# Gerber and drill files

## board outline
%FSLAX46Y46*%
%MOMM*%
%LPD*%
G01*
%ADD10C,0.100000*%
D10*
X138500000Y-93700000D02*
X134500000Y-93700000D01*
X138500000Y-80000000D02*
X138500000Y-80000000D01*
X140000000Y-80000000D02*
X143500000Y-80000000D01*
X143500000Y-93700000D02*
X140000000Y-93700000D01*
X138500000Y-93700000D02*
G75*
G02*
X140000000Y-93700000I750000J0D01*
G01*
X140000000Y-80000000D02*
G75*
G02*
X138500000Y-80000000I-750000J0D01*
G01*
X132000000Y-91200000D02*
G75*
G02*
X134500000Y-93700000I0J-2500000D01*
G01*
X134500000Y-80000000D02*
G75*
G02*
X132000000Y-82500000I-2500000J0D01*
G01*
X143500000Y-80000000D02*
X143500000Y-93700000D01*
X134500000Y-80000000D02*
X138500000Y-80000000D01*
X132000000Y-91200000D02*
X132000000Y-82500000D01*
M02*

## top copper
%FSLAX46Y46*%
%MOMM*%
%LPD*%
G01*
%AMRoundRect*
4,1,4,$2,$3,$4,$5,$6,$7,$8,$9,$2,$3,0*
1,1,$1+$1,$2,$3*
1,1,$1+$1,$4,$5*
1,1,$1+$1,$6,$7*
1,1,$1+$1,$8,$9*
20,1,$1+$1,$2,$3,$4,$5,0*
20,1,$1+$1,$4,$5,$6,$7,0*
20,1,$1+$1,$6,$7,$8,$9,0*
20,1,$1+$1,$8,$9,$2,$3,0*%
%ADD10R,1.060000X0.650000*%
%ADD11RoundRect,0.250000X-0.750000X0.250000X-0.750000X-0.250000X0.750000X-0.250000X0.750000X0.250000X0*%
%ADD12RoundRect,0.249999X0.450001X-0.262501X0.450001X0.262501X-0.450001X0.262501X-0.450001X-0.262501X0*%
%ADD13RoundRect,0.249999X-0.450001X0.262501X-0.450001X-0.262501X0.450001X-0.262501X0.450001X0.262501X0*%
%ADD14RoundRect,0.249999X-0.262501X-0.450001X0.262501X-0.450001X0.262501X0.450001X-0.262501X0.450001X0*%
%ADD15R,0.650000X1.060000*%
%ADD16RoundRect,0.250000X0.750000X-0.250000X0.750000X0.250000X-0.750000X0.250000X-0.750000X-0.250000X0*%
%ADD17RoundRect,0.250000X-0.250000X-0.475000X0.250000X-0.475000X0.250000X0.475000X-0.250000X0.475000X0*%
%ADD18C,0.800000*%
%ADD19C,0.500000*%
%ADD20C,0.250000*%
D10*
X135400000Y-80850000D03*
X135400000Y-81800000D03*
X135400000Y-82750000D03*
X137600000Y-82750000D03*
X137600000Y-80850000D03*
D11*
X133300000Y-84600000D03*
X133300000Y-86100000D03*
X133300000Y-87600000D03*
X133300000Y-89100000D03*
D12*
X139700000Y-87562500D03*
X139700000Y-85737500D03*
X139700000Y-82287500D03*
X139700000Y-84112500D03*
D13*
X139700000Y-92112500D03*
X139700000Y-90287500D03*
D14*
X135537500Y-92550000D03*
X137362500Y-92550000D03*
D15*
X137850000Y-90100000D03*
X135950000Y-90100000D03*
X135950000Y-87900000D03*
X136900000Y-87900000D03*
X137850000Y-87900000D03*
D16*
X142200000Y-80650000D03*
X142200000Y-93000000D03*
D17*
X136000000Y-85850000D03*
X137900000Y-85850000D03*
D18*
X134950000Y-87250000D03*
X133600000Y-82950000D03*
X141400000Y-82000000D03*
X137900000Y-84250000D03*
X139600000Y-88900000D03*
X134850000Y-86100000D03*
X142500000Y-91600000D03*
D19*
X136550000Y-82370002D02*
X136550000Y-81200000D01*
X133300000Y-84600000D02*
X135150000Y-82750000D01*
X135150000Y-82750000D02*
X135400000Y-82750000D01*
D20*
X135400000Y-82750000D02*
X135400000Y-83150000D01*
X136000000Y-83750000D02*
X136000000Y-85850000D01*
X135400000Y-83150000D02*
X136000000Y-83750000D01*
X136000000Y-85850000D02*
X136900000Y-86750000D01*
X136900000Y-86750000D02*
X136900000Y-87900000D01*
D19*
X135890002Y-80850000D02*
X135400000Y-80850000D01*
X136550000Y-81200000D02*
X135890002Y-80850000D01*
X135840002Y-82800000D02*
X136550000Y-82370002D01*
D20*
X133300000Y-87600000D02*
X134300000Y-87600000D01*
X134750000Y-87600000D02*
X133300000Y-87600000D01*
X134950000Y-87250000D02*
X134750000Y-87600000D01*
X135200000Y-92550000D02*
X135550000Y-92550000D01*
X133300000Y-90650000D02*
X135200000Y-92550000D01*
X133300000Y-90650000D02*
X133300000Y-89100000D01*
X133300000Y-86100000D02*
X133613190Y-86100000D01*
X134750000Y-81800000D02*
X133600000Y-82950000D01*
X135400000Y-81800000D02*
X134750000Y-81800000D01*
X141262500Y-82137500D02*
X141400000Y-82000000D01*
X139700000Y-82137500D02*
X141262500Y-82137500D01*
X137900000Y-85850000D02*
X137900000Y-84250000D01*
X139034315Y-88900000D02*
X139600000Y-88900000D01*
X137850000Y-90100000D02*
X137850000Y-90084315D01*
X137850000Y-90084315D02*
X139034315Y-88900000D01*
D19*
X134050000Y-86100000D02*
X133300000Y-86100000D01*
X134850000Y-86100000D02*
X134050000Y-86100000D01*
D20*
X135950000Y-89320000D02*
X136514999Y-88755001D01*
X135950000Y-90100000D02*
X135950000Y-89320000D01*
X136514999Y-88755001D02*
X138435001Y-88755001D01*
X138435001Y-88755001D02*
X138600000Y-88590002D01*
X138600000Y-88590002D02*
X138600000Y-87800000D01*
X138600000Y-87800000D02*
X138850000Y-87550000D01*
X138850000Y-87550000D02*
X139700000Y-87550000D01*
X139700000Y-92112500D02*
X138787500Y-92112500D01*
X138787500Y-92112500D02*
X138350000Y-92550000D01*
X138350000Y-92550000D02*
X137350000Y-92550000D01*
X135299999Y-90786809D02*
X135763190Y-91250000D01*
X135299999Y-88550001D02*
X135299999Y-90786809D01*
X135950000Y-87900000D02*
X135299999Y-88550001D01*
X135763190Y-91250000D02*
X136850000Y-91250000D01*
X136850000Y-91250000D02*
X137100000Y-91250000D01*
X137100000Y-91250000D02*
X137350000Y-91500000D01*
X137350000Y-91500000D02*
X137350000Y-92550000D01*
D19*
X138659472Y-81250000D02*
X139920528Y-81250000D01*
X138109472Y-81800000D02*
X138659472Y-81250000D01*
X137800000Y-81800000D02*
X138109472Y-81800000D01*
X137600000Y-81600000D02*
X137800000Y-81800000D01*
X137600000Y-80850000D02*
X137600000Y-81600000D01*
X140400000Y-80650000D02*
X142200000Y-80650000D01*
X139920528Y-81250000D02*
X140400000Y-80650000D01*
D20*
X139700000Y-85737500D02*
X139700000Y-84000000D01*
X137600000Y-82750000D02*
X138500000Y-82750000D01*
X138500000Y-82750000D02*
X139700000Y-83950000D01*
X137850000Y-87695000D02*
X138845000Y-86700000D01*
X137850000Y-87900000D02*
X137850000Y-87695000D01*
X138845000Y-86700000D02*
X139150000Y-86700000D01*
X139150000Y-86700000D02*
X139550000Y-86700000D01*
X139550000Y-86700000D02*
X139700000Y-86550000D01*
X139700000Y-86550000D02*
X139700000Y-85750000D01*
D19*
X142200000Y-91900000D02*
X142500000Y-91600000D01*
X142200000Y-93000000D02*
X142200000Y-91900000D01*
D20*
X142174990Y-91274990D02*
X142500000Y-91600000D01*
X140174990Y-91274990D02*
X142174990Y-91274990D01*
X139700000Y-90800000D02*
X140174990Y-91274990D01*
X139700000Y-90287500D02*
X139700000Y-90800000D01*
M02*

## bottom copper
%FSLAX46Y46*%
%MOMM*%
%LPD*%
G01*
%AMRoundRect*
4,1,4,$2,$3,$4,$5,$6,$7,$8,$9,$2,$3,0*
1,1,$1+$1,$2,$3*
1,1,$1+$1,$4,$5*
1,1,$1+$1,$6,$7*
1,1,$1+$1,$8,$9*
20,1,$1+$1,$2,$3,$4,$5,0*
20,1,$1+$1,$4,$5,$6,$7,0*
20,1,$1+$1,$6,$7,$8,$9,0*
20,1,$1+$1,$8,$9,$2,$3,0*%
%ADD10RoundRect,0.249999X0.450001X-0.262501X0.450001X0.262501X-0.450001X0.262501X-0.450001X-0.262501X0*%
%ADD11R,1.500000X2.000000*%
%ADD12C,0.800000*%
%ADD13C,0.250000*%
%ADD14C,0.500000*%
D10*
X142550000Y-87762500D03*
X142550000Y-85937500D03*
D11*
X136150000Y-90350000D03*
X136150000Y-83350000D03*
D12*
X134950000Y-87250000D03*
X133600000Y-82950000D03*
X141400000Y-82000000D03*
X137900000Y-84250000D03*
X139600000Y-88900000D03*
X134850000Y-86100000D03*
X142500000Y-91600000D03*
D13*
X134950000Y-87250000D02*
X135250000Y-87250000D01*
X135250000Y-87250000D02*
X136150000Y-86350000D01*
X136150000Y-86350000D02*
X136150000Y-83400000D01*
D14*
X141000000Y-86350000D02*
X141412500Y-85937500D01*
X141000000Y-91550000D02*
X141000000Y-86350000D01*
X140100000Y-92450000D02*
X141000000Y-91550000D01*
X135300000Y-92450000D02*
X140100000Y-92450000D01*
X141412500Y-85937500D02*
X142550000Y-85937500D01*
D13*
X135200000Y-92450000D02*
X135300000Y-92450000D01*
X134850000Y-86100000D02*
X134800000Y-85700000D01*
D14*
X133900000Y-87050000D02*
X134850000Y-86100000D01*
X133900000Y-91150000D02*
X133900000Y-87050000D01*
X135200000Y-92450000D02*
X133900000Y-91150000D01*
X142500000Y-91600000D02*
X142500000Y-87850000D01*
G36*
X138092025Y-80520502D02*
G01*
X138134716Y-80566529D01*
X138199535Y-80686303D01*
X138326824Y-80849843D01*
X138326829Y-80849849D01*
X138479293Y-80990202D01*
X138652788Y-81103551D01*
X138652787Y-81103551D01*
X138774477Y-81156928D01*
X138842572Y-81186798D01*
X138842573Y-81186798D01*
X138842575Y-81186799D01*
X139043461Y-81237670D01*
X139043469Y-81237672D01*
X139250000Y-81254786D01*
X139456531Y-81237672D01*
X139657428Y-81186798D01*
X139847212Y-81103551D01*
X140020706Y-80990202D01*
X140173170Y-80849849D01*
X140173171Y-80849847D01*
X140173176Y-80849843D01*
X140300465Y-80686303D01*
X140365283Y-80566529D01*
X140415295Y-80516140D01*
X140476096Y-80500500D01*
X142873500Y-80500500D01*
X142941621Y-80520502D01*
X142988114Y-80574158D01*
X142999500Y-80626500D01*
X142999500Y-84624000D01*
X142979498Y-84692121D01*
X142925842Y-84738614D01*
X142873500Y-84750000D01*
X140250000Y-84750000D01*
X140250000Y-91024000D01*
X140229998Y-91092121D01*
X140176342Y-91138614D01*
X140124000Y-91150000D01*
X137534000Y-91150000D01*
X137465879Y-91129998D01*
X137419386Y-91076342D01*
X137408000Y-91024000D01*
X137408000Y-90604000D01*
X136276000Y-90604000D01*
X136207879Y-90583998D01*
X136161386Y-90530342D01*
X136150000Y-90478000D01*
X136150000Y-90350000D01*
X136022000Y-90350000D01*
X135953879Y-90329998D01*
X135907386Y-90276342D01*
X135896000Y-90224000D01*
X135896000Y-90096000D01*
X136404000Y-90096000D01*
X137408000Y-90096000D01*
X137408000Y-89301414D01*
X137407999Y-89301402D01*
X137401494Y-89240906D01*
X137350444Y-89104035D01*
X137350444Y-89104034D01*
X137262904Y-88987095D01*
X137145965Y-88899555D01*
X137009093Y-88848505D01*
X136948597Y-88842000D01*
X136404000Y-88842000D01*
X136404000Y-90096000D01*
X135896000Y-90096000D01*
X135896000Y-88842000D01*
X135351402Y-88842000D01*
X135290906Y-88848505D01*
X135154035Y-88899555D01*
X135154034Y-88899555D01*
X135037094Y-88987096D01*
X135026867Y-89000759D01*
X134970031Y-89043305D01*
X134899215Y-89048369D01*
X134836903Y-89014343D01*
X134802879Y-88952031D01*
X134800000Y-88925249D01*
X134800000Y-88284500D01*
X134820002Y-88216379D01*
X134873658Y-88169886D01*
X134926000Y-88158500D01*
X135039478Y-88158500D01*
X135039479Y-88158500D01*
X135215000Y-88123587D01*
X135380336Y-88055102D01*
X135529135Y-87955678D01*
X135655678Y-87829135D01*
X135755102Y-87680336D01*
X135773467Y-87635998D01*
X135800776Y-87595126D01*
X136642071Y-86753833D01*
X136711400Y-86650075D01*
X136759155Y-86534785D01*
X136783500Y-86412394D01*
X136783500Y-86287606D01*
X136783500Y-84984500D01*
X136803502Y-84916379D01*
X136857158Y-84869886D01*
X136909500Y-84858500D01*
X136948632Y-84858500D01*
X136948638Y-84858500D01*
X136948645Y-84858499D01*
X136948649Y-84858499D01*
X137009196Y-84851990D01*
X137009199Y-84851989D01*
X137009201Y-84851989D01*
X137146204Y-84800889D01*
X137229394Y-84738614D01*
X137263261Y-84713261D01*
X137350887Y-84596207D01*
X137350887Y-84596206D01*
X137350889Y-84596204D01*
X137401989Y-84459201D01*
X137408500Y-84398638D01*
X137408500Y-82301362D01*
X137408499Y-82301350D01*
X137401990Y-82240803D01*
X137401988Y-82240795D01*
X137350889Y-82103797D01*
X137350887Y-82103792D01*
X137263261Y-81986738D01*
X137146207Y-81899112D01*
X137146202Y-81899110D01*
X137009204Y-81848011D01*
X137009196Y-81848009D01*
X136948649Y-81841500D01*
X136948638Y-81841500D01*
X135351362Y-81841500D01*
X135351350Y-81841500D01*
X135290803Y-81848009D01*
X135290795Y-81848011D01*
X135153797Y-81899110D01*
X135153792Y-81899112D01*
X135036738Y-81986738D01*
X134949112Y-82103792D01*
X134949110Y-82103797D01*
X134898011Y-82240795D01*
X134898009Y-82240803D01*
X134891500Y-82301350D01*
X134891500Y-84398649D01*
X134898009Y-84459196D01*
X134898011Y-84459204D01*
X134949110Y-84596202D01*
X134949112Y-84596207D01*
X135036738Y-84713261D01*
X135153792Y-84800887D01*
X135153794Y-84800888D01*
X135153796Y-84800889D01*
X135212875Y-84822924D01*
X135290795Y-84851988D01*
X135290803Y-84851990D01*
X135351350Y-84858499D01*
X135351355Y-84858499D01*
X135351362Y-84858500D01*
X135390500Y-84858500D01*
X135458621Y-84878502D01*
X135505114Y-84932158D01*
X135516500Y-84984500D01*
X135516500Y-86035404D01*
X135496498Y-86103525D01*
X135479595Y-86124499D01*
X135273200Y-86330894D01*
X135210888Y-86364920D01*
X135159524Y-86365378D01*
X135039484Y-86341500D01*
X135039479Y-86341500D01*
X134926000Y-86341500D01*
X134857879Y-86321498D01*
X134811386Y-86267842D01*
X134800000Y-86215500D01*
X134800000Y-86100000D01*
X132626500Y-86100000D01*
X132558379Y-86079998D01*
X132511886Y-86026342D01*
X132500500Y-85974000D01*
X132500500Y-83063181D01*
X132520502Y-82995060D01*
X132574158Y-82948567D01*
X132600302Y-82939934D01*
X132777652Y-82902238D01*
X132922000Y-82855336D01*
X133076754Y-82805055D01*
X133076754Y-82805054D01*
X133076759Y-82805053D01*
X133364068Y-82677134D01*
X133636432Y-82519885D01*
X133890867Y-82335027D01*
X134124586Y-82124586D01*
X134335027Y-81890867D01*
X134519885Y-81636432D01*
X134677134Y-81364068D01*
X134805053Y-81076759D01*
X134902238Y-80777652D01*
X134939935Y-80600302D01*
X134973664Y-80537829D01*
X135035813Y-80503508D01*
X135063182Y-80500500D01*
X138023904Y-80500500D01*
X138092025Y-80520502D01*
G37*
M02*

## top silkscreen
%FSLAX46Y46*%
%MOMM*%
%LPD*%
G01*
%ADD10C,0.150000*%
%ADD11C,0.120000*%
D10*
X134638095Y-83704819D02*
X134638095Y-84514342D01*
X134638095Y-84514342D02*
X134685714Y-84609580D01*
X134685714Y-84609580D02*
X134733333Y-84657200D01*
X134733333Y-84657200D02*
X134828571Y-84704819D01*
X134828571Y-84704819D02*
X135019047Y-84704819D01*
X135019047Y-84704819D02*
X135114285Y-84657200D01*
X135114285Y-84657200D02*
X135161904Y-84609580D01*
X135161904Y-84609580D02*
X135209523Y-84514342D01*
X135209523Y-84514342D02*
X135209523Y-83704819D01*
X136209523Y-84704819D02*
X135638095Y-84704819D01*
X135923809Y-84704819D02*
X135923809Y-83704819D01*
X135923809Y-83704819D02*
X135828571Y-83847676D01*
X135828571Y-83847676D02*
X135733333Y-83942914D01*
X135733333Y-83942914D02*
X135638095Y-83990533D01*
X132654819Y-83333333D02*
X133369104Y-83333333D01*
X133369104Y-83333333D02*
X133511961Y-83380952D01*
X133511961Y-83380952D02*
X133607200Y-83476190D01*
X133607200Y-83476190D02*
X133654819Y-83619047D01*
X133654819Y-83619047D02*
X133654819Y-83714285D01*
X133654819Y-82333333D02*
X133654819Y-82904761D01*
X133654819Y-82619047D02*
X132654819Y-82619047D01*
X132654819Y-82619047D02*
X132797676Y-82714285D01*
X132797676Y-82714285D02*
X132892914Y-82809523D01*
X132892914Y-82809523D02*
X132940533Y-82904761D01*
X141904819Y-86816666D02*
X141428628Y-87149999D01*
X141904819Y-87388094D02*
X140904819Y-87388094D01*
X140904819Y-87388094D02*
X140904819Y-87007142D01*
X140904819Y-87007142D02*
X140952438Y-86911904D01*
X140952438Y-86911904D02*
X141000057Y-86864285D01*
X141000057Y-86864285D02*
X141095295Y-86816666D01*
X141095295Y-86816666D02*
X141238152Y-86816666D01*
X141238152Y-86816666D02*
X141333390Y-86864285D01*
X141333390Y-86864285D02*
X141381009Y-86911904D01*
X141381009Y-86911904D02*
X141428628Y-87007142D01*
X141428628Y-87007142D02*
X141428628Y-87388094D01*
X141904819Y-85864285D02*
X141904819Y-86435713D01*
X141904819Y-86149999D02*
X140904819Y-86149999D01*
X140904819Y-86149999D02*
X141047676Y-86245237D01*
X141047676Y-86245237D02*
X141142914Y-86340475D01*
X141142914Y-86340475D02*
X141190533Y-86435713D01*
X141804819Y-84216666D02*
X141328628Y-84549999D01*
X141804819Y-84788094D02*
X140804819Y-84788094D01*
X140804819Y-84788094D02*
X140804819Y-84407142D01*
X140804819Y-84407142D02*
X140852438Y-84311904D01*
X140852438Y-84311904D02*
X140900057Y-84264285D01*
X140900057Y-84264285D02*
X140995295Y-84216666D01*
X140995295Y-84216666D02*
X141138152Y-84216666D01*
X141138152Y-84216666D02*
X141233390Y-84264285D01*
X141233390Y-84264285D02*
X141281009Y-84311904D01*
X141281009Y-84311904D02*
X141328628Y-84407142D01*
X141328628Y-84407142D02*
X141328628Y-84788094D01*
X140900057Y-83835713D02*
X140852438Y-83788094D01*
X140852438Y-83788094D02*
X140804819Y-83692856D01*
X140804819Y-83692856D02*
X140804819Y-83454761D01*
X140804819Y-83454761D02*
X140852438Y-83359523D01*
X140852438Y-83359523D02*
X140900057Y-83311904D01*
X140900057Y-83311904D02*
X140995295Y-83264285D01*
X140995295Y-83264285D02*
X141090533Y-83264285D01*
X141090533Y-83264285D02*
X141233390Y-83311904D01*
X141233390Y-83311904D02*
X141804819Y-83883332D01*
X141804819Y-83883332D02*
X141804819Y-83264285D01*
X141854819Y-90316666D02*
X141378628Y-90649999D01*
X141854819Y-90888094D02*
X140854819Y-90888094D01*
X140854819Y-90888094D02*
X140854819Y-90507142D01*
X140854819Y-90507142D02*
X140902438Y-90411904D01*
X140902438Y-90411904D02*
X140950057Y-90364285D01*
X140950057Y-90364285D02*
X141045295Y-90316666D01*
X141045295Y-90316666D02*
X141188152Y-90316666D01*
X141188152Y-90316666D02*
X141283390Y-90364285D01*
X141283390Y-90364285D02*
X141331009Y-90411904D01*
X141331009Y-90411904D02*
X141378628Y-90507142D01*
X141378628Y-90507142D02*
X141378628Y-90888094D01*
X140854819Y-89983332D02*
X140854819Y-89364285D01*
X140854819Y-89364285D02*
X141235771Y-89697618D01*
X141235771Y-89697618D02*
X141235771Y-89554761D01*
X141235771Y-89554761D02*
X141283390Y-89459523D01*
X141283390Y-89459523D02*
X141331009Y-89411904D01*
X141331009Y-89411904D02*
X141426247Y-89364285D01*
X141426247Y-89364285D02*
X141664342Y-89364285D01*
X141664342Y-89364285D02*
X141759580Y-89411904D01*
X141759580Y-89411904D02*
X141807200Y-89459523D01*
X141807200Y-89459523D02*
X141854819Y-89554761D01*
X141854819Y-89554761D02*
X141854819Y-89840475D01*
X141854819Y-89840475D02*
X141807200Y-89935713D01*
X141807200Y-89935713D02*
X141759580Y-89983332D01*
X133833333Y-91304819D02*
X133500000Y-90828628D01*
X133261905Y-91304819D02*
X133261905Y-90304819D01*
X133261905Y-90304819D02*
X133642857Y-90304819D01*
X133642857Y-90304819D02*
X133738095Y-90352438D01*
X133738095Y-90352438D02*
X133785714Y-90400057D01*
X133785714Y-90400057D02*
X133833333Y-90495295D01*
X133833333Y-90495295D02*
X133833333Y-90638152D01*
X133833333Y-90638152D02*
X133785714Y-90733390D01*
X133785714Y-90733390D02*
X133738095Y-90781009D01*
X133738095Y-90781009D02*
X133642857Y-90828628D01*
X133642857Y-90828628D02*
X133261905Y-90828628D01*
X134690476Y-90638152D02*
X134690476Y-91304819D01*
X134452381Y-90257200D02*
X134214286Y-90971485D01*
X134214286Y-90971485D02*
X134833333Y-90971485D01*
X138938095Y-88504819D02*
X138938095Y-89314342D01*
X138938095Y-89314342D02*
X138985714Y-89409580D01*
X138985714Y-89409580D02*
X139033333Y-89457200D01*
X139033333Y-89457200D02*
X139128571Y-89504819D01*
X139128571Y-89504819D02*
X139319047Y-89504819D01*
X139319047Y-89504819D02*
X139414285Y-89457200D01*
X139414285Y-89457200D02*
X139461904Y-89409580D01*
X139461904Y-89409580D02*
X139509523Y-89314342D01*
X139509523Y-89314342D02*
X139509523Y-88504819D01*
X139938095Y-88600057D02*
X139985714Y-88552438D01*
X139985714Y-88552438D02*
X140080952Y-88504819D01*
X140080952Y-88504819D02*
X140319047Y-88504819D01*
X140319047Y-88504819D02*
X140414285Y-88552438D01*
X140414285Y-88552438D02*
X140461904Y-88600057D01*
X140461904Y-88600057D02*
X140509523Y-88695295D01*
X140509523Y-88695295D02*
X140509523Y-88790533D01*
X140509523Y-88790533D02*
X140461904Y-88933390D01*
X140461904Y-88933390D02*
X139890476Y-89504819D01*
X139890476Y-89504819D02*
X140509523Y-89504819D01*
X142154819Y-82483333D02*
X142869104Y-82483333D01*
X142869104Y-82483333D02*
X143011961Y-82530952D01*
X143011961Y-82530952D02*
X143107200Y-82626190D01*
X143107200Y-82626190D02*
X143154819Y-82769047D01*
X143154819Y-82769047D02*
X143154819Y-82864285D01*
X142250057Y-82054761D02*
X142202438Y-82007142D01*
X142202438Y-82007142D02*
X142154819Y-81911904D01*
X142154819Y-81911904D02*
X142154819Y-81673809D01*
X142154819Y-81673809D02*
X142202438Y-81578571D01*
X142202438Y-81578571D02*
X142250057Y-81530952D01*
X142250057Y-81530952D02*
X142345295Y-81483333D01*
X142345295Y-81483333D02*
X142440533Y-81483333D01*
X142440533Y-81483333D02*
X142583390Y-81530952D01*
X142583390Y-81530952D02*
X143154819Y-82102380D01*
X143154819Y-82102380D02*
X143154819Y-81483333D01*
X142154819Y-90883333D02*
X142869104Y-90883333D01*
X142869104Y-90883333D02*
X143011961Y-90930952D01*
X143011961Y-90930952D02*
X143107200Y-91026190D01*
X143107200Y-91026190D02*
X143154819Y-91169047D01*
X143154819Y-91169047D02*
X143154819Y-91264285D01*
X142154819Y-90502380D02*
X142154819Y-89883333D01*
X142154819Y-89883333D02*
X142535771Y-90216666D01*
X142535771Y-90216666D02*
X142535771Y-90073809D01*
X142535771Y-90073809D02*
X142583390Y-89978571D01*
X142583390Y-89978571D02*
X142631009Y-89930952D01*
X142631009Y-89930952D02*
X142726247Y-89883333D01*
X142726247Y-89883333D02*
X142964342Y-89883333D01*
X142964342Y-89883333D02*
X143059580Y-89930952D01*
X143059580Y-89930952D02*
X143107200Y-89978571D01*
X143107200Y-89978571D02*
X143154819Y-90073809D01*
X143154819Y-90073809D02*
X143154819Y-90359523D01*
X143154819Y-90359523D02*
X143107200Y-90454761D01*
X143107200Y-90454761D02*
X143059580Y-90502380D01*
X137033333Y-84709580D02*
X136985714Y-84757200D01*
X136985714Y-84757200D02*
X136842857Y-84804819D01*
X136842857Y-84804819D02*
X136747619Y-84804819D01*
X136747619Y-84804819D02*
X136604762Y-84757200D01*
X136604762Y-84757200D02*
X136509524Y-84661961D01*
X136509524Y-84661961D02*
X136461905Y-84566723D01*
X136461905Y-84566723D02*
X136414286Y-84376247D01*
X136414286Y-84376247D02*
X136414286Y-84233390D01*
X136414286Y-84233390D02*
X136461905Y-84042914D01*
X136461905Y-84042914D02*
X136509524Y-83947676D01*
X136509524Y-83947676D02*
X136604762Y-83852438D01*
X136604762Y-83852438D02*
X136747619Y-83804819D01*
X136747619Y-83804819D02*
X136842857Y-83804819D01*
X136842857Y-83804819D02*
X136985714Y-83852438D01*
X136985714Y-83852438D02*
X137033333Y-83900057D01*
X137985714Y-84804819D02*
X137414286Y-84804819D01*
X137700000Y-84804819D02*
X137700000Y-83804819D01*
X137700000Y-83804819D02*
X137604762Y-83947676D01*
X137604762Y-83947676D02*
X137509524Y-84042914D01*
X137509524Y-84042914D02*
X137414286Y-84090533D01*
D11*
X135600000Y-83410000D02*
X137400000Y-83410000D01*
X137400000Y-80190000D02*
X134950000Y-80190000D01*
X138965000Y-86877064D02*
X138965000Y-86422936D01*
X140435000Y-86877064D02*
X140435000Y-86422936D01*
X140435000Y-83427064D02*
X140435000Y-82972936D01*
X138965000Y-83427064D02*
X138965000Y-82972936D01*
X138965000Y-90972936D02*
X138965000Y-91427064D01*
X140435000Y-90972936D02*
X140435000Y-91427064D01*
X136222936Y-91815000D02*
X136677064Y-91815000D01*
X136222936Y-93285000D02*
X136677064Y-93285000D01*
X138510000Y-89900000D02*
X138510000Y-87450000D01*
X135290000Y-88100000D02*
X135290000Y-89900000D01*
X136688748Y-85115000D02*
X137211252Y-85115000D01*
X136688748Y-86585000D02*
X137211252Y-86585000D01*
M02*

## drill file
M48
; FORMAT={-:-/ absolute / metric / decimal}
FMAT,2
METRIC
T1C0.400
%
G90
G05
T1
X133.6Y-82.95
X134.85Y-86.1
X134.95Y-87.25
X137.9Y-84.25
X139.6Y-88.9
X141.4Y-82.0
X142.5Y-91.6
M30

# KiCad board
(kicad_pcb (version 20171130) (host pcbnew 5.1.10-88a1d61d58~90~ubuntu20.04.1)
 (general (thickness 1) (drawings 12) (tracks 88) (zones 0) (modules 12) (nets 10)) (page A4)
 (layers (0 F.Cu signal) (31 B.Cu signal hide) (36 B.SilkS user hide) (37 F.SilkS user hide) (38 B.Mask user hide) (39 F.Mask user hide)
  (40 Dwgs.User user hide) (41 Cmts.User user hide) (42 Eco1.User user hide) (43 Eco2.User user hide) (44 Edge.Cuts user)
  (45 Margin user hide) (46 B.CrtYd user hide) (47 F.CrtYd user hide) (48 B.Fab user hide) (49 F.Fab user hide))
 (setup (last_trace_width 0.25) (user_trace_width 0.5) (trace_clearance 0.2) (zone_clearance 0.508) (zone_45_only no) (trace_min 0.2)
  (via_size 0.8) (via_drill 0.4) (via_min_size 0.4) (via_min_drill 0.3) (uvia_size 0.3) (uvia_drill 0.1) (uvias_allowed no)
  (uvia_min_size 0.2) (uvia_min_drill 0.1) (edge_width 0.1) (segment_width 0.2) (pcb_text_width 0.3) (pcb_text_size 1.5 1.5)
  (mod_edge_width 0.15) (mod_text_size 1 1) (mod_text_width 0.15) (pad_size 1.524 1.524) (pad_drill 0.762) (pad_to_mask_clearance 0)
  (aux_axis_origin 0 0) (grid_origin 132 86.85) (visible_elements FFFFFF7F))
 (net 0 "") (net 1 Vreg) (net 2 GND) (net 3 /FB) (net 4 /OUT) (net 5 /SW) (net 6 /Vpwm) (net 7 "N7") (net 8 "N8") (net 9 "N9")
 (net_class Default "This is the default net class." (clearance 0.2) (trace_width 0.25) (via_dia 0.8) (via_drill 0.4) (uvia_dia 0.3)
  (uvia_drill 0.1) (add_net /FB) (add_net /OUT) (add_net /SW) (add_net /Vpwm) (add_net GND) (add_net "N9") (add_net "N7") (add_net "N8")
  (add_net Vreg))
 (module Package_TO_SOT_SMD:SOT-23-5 (layer F.Cu) (at 136.5 81.8)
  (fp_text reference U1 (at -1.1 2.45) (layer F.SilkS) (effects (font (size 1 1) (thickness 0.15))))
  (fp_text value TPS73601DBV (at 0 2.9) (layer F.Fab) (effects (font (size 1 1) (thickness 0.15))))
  (fp_line (start -0.9 1.61) (end 0.9 1.61) (layer F.SilkS) (width 0.12))
  (fp_line (start 0.9 -1.61) (end -1.55 -1.61) (layer F.SilkS) (width 0.12))
  (pad 1 smd rect (at -1.1 -0.95) (size 1.06 0.65) (layers F.Cu F.Paste F.Mask) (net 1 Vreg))
  (pad 2 smd rect (at -1.1 0) (size 1.06 0.65) (layers F.Cu F.Paste F.Mask) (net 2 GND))
  (pad 3 smd rect (at -1.1 0.95) (size 1.06 0.65) (layers F.Cu F.Paste F.Mask) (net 1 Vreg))
  (pad 4 smd rect (at 1.1 0.95) (size 1.06 0.65) (layers F.Cu F.Paste F.Mask) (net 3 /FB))
  (pad 5 smd rect (at 1.1 -0.95) (size 1.06 0.65) (layers F.Cu F.Paste F.Mask) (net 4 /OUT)))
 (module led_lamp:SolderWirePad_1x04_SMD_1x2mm (layer F.Cu) (at 133.3 84.6 270)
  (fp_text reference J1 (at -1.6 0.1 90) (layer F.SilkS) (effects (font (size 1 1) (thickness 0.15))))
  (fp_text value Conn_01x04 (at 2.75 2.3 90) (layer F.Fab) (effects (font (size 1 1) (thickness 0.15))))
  (pad 1 smd roundrect (at 0 0 270) (size 1 2) (layers F.Cu F.Paste F.Mask) (roundrect_rratio 0.25) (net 1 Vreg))
  (pad 2 smd roundrect (at 1.5 0 270) (size 1 2) (layers F.Cu F.Paste F.Mask) (roundrect_rratio 0.25) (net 2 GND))
  (pad 3 smd roundrect (at 3 0 270) (size 1 2) (layers F.Cu F.Paste F.Mask) (roundrect_rratio 0.25) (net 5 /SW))
  (pad 4 smd roundrect (at 4.5 0 270) (size 1 2) (layers F.Cu F.Paste F.Mask) (roundrect_rratio 0.25) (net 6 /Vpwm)))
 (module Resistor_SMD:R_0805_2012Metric (layer F.Cu) (at 139.7 86.65 90)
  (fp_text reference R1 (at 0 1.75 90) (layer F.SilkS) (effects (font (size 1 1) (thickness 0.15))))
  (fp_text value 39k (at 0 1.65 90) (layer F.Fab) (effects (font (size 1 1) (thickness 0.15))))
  (fp_line (start -0.227064 -0.735) (end 0.227064 -0.735) (layer F.SilkS) (width 0.12))
  (fp_line (start -0.227064 0.735) (end 0.227064 0.735) (layer F.SilkS) (width 0.12))
  (pad 1 smd roundrect (at -0.9125 0 90) (size 1.025 1.4) (layers F.Cu F.Paste F.Mask) (roundrect_rratio 0.2439014634146341) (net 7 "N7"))
  (pad 2 smd roundrect (at 0.9125 0 90) (size 1.025 1.4) (layers F.Cu F.Paste F.Mask) (roundrect_rratio 0.2439014634146341) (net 3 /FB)))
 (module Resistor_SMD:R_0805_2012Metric (layer F.Cu) (at 139.7 83.2 90)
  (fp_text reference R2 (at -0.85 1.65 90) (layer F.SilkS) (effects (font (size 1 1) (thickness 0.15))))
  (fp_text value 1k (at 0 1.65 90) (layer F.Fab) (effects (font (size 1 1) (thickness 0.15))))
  (fp_line (start -0.227064 0.735) (end 0.227064 0.735) (layer F.SilkS) (width 0.12))
  (fp_line (start -0.227064 -0.735) (end 0.227064 -0.735) (layer F.SilkS) (width 0.12))
  (pad 2 smd roundrect (at 0.9125 0 90) (size 1.025 1.4) (layers F.Cu F.Paste F.Mask) (roundrect_rratio 0.2439014634146341) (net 2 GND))
  (pad 1 smd roundrect (at -0.9125 0 90) (size 1.025 1.4) (layers F.Cu F.Paste F.Mask) (roundrect_rratio 0.2439014634146341) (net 3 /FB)))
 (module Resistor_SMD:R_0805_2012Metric (layer F.Cu) (at 139.7 91.2 270)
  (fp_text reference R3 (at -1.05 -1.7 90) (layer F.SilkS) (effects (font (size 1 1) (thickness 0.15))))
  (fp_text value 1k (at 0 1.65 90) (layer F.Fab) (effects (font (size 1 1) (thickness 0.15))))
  (fp_line (start -0.227064 0.735) (end 0.227064 0.735) (layer F.SilkS) (width 0.12))
  (fp_line (start -0.227064 -0.735) (end 0.227064 -0.735) (layer F.SilkS) (width 0.12))
  (pad 2 smd roundrect (at 0.9125 0 270) (size 1.025 1.4) (layers F.Cu F.Paste F.Mask) (roundrect_rratio 0.2439014634146341) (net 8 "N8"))
  (pad 1 smd roundrect (at -0.9125 0 270) (size 1.025 1.4) (layers F.Cu F.Paste F.Mask) (roundrect_rratio 0.2439014634146341) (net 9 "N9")))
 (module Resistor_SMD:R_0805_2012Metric (layer F.Cu) (at 136.45 92.55)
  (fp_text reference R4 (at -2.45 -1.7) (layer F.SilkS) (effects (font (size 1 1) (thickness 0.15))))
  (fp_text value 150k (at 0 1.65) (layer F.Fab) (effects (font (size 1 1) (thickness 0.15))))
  (fp_line (start -0.227064 -0.735) (end 0.227064 -0.735) (layer F.SilkS) (width 0.12))
  (fp_line (start -0.227064 0.735) (end 0.227064 0.735) (layer F.SilkS) (width 0.12))
  (pad 1 smd roundrect (at -0.9125 0) (size 1.025 1.4) (layers F.Cu F.Paste F.Mask) (roundrect_rratio 0.2439014634146341) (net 6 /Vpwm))
  (pad 2 smd roundrect (at 0.9125 0) (size 1.025 1.4) (layers F.Cu F.Paste F.Mask) (roundrect_rratio 0.2439014634146341) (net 8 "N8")))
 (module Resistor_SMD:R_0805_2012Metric (layer B.Cu) (at 142.55 86.85 90)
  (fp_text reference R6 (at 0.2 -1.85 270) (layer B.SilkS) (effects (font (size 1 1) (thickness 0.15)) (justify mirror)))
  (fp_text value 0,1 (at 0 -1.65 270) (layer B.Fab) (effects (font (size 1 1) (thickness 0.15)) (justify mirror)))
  (pad 1 smd roundrect (at -0.9125 0 90) (size 1.025 1.4) (layers B.Cu B.Paste B.Mask) (roundrect_rratio 0.2439014634146341) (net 9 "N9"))
  (pad 2 smd roundrect (at 0.9125 0 90) (size 1.025 1.4) (layers B.Cu B.Paste B.Mask) (roundrect_rratio 0.2439014634146341) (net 2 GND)))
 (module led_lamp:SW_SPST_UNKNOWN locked (layer B.Cu) (at 136.15 86.85 90)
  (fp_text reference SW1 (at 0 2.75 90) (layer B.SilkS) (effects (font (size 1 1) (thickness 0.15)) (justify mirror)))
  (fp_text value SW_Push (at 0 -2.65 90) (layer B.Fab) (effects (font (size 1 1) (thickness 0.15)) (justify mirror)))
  (pad 1 smd rect (at -3.5 0 90) (size 2 1.5) (layers B.Cu B.Paste B.Mask) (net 2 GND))
  (pad 2 smd rect (at 3.5 0 90) (size 2 1.5) (layers B.Cu B.Paste B.Mask) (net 5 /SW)))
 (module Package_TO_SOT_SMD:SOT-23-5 (layer F.Cu) (at 136.9 89 270)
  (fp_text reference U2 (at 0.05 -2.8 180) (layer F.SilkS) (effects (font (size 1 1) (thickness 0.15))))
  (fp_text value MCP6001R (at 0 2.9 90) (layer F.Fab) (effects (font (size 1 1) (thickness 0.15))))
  (fp_line (start 0.9 -1.61) (end -1.55 -1.61) (layer F.SilkS) (width 0.12))
  (fp_line (start -0.9 1.61) (end 0.9 1.61) (layer F.SilkS) (width 0.12))
  (pad 5 smd rect (at 1.1 -0.95 270) (size 1.06 0.65) (layers F.Cu F.Paste F.Mask) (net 2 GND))
  (pad 4 smd rect (at 1.1 0.95 270) (size 1.06 0.65) (layers F.Cu F.Paste F.Mask) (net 7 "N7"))
  (pad 3 smd rect (at -1.1 0.95 270) (size 1.06 0.65) (layers F.Cu F.Paste F.Mask) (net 8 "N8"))
  (pad 2 smd rect (at -1.1 0 270) (size 1.06 0.65) (layers F.Cu F.Paste F.Mask) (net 1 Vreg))
  (pad 1 smd rect (at -1.1 -0.95 270) (size 1.06 0.65) (layers F.Cu F.Paste F.Mask) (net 3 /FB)))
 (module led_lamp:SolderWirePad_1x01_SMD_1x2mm (layer F.Cu) (at 142.2 80.65 90)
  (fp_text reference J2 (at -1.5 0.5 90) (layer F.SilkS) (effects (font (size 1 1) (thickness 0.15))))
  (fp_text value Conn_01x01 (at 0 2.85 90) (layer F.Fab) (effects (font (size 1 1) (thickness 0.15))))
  (pad 1 smd roundrect (at 0 0 90) (size 1 2) (layers F.Cu F.Paste F.Mask) (roundrect_rratio 0.25) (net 4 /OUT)))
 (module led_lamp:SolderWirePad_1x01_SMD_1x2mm (layer F.Cu) (at 142.2 93 90)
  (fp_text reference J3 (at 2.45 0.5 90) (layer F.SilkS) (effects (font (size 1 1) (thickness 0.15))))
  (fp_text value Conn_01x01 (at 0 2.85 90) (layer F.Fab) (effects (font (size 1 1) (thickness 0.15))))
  (pad 1 smd roundrect (at 0 0 90) (size 1 2) (layers F.Cu F.Paste F.Mask) (roundrect_rratio 0.25) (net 9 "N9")))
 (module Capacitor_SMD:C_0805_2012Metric (layer F.Cu) (at 136.95 85.85)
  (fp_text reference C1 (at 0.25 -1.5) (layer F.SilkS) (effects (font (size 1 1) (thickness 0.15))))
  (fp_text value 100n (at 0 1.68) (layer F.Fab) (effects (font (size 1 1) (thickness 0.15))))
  (fp_line (start -0.261252 -0.735) (end 0.261252 -0.735) (layer F.SilkS) (width 0.12))
  (fp_line (start -0.261252 0.735) (end 0.261252 0.735) (layer F.SilkS) (width 0.12))
  (pad 1 smd roundrect (at -0.95 0) (size 1 1.45) (layers F.Cu F.Paste F.Mask) (roundrect_rratio 0.25) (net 1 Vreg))
  (pad 2 smd roundrect (at 0.95 0) (size 1 1.45) (layers F.Cu F.Paste F.Mask) (roundrect_rratio 0.25) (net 2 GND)))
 (gr_line (start 138.5 93.7) (end 134.5 93.7) (layer Edge.Cuts) (width 0.1))
 (gr_line (start 138.5 80) (end 138.5 80) (layer Edge.Cuts) (width 0.1))
 (gr_line (start 140 80) (end 143.5 80) (layer Edge.Cuts) (width 0.1))
 (gr_line (start 143.5 93.7) (end 140 93.7) (layer Edge.Cuts) (width 0.1))
 (gr_arc (start 139.25 93.7) (end 140 93.7) (angle -180) (layer Edge.Cuts) (width 0.1))
 (gr_arc (start 139.25 80) (end 138.5 80) (angle -180) (layer Edge.Cuts) (width 0.1))
 (gr_arc (start 132 93.7) (end 134.5 93.7) (angle -90) (layer Edge.Cuts) (width 0.1))
 (gr_arc (start 132 80) (end 132 82.5) (angle -90) (layer Edge.Cuts) (width 0.1))
 (gr_line (start 143.5 80) (end 143.5 93.7) (layer Edge.Cuts) (width 0.1))
 (gr_line (start 134.5 80) (end 138.5 80) (layer Edge.Cuts) (width 0.1))
 (gr_line (start 132 91.2) (end 132 82.5) (layer Edge.Cuts) (width 0.1))
 (segment (start 136.55 82.370002) (end 136.55 81.2) (width 0.5) (layer F.Cu) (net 1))
 (segment (start 133.3 84.6) (end 135.15 82.75) (width 0.5) (layer F.Cu) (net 1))
 (segment (start 135.15 82.75) (end 135.4 82.75) (width 0.5) (layer F.Cu) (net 1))
 (segment (start 135.4 82.75) (end 135.4 83.15) (width 0.25) (layer F.Cu) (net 1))
 (segment (start 136 83.75) (end 136 85.85) (width 0.25) (layer F.Cu) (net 1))
 (segment (start 135.4 83.15) (end 136 83.75) (width 0.25) (layer F.Cu) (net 1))
 (segment (start 136 85.85) (end 136.9 86.75) (width 0.25) (layer F.Cu) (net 1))
 (segment (start 136.9 86.75) (end 136.9 87.9) (width 0.25) (layer F.Cu) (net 1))
 (segment (start 135.890002 80.85) (end 135.4 80.85) (width 0.5) (layer F.Cu) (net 1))
 (segment (start 136.55 81.2) (end 135.890002 80.85) (width 0.5) (layer F.Cu) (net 1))
 (segment (start 135.840002 82.8) (end 136.55 82.370002) (width 0.5) (layer F.Cu) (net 1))
 (segment (start 133.3 87.6) (end 134.3 87.6) (width 0.25) (layer F.Cu) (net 5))
 (segment (start 134.75 87.6) (end 133.3 87.6) (width 0.25) (layer F.Cu) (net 5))
 (segment (start 134.95 87.25) (end 135.25 87.25) (width 0.25) (layer B.Cu) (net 5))
 (segment (start 135.25 87.25) (end 136.15 86.35) (width 0.25) (layer B.Cu) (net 5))
 (segment (start 136.15 86.35) (end 136.15 83.4) (width 0.25) (layer B.Cu) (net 5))
 (via (at 134.95 87.25) (size 0.8) (drill 0.4) (layers F.Cu B.Cu) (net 5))
 (segment (start 134.95 87.25) (end 134.75 87.6) (width 0.25) (layer F.Cu) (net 5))
 (segment (start 135.2 92.55) (end 135.55 92.55) (width 0.25) (layer F.Cu) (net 6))
 (segment (start 133.3 90.65) (end 135.2 92.55) (width 0.25) (layer F.Cu) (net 6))
 (segment (start 133.3 90.65) (end 133.3 89.1) (width 0.25) (layer F.Cu) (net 6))
 (segment (start 133.3 86.1) (end 133.61319 86.1) (width 0.25) (layer F.Cu) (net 2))
 (via (at 133.6 82.95) (size 0.8) (drill 0.4) (layers F.Cu B.Cu) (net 2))
 (segment (start 134.75 81.8) (end 133.6 82.95) (width 0.25) (layer F.Cu) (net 2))
 (segment (start 135.4 81.8) (end 134.75 81.8) (width 0.25) (layer F.Cu) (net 2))
 (via (at 141.4 82) (size 0.8) (drill 0.4) (layers F.Cu B.Cu) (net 2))
 (segment (start 141.2625 82.1375) (end 141.4 82) (width 0.25) (layer F.Cu) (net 2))
 (segment (start 139.7 82.1375) (end 141.2625 82.1375) (width 0.25) (layer F.Cu) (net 2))
 (via (at 137.9 84.25) (size 0.8) (drill 0.4) (layers F.Cu B.Cu) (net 2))
 (segment (start 137.9 85.85) (end 137.9 84.25) (width 0.25) (layer F.Cu) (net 2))
 (via (at 139.6 88.9) (size 0.8) (drill 0.4) (layers F.Cu B.Cu) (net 2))
 (segment (start 139.034315 88.9) (end 139.6 88.9) (width 0.25) (layer F.Cu) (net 2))
 (segment (start 137.85 90.1) (end 137.85 90.084315) (width 0.25) (layer F.Cu) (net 2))
 (segment (start 137.85 90.084315) (end 139.034315 88.9) (width 0.25) (layer F.Cu) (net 2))
 (segment (start 141 86.35) (end 141.4125 85.9375) (width 0.5) (layer B.Cu) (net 2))
 (segment (start 141 91.55) (end 141 86.35) (width 0.5) (layer B.Cu) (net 2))
 (segment (start 140.1 92.45) (end 141 91.55) (width 0.5) (layer B.Cu) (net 2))
 (segment (start 135.3 92.45) (end 140.1 92.45) (width 0.5) (layer B.Cu) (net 2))
 (segment (start 141.4125 85.9375) (end 142.55 85.9375) (width 0.5) (layer B.Cu) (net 2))
 (segment (start 135.2 92.45) (end 135.3 92.45) (width 0.25) (layer B.Cu) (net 2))
 (segment (start 134.85 86.1) (end 134.8 85.7) (width 0.25) (layer B.Cu) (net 2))
 (segment (start 134.05 86.1) (end 133.3 86.1) (width 0.5) (layer F.Cu) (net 2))
 (segment (start 134.85 86.1) (end 134.05 86.1) (width 0.5) (layer F.Cu) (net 2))
 (via (at 134.85 86.1) (size 0.8) (drill 0.4) (layers F.Cu B.Cu) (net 2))
 (segment (start 133.9 87.05) (end 134.85 86.1) (width 0.5) (layer B.Cu) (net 2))
 (segment (start 133.9 91.15) (end 133.9 87.05) (width 0.5) (layer B.Cu) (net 2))
 (segment (start 135.2 92.45) (end 133.9 91.15) (width 0.5) (layer B.Cu) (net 2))
 (segment (start 135.95 89.32) (end 136.514999 88.755001) (width 0.25) (layer F.Cu) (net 7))
 (segment (start 135.95 90.1) (end 135.95 89.32) (width 0.25) (layer F.Cu) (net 7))
 (segment (start 136.514999 88.755001) (end 138.435001 88.755001) (width 0.25) (layer F.Cu) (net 7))
 (segment (start 138.435001 88.755001) (end 138.6 88.590002) (width 0.25) (layer F.Cu) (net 7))
 (segment (start 138.6 88.590002) (end 138.6 87.8) (width 0.25) (layer F.Cu) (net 7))
 (segment (start 138.6 87.8) (end 138.85 87.55) (width 0.25) (layer F.Cu) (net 7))
 (segment (start 138.85 87.55) (end 139.7 87.55) (width 0.25) (layer F.Cu) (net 7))
 (segment (start 139.7 92.1125) (end 138.7875 92.1125) (width 0.25) (layer F.Cu) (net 8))
 (segment (start 138.7875 92.1125) (end 138.35 92.55) (width 0.25) (layer F.Cu) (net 8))
 (segment (start 138.35 92.55) (end 137.35 92.55) (width 0.25) (layer F.Cu) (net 8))
 (segment (start 135.299999 90.786809) (end 135.76319 91.25) (width 0.25) (layer F.Cu) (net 8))
 (segment (start 135.299999 88.550001) (end 135.299999 90.786809) (width 0.25) (layer F.Cu) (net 8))
 (segment (start 135.95 87.9) (end 135.299999 88.550001) (width 0.25) (layer F.Cu) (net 8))
 (segment (start 135.76319 91.25) (end 136.85 91.25) (width 0.25) (layer F.Cu) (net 8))
 (segment (start 136.85 91.25) (end 137.1 91.25) (width 0.25) (layer F.Cu) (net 8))
 (segment (start 137.1 91.25) (end 137.35 91.5) (width 0.25) (layer F.Cu) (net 8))
 (segment (start 137.35 91.5) (end 137.35 92.55) (width 0.25) (layer F.Cu) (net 8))
 (segment (start 138.659472 81.25) (end 139.920528 81.25) (width 0.5) (layer F.Cu) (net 4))
 (segment (start 138.109472 81.8) (end 138.659472 81.25) (width 0.5) (layer F.Cu) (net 4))
 (segment (start 137.8 81.8) (end 138.109472 81.8) (width 0.5) (layer F.Cu) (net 4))
 (segment (start 137.6 81.6) (end 137.8 81.8) (width 0.5) (layer F.Cu) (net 4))
 (segment (start 137.6 80.85) (end 137.6 81.6) (width 0.5) (layer F.Cu) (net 4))
 (segment (start 140.4 80.65) (end 142.2 80.65) (width 0.5) (layer F.Cu) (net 4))
 (segment (start 139.920528 81.25) (end 140.4 80.65) (width 0.5) (layer F.Cu) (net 4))
 (segment (start 139.7 85.7375) (end 139.7 84) (width 0.25) (layer F.Cu) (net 3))
 (segment (start 137.6 82.75) (end 138.5 82.75) (width 0.25) (layer F.Cu) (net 3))
 (segment (start 138.5 82.75) (end 139.7 83.95) (width 0.25) (layer F.Cu) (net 3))
 (segment (start 137.85 87.695) (end 138.845 86.7) (width 0.25) (layer F.Cu) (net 3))
 (segment (start 137.85 87.9) (end 137.85 87.695) (width 0.25) (layer F.Cu) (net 3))
 (segment (start 138.845 86.7) (end 139.15 86.7) (width 0.25) (layer F.Cu) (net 3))
 (segment (start 139.15 86.7) (end 139.55 86.7) (width 0.25) (layer F.Cu) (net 3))
 (segment (start 139.55 86.7) (end 139.7 86.55) (width 0.25) (layer F.Cu) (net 3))
 (segment (start 139.7 86.55) (end 139.7 85.75) (width 0.25) (layer F.Cu) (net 3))
 (via (at 142.5 91.6) (size 0.8) (drill 0.4) (layers F.Cu B.Cu) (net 9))
 (segment (start 142.2 91.9) (end 142.5 91.6) (width 0.5) (layer F.Cu) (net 9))
 (segment (start 142.2 93) (end 142.2 91.9) (width 0.5) (layer F.Cu) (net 9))
 (segment (start 142.5 91.6) (end 142.5 87.85) (width 0.5) (layer B.Cu) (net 9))
 (segment (start 142.17499 91.27499) (end 142.5 91.6) (width 0.25) (layer F.Cu) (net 9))
 (segment (start 140.17499 91.27499) (end 142.17499 91.27499) (width 0.25) (layer F.Cu) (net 9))
 (segment (start 139.7 90.8) (end 140.17499 91.27499) (width 0.25) (layer F.Cu) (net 9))
 (segment (start 139.7 90.2875) (end 139.7 90.8) (width 0.25) (layer F.Cu) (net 9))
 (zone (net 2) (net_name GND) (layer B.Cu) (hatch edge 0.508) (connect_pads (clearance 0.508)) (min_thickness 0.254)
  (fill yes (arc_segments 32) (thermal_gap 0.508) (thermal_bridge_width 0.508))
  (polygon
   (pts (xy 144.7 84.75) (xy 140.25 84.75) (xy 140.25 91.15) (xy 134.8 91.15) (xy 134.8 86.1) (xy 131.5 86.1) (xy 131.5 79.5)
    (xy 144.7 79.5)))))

